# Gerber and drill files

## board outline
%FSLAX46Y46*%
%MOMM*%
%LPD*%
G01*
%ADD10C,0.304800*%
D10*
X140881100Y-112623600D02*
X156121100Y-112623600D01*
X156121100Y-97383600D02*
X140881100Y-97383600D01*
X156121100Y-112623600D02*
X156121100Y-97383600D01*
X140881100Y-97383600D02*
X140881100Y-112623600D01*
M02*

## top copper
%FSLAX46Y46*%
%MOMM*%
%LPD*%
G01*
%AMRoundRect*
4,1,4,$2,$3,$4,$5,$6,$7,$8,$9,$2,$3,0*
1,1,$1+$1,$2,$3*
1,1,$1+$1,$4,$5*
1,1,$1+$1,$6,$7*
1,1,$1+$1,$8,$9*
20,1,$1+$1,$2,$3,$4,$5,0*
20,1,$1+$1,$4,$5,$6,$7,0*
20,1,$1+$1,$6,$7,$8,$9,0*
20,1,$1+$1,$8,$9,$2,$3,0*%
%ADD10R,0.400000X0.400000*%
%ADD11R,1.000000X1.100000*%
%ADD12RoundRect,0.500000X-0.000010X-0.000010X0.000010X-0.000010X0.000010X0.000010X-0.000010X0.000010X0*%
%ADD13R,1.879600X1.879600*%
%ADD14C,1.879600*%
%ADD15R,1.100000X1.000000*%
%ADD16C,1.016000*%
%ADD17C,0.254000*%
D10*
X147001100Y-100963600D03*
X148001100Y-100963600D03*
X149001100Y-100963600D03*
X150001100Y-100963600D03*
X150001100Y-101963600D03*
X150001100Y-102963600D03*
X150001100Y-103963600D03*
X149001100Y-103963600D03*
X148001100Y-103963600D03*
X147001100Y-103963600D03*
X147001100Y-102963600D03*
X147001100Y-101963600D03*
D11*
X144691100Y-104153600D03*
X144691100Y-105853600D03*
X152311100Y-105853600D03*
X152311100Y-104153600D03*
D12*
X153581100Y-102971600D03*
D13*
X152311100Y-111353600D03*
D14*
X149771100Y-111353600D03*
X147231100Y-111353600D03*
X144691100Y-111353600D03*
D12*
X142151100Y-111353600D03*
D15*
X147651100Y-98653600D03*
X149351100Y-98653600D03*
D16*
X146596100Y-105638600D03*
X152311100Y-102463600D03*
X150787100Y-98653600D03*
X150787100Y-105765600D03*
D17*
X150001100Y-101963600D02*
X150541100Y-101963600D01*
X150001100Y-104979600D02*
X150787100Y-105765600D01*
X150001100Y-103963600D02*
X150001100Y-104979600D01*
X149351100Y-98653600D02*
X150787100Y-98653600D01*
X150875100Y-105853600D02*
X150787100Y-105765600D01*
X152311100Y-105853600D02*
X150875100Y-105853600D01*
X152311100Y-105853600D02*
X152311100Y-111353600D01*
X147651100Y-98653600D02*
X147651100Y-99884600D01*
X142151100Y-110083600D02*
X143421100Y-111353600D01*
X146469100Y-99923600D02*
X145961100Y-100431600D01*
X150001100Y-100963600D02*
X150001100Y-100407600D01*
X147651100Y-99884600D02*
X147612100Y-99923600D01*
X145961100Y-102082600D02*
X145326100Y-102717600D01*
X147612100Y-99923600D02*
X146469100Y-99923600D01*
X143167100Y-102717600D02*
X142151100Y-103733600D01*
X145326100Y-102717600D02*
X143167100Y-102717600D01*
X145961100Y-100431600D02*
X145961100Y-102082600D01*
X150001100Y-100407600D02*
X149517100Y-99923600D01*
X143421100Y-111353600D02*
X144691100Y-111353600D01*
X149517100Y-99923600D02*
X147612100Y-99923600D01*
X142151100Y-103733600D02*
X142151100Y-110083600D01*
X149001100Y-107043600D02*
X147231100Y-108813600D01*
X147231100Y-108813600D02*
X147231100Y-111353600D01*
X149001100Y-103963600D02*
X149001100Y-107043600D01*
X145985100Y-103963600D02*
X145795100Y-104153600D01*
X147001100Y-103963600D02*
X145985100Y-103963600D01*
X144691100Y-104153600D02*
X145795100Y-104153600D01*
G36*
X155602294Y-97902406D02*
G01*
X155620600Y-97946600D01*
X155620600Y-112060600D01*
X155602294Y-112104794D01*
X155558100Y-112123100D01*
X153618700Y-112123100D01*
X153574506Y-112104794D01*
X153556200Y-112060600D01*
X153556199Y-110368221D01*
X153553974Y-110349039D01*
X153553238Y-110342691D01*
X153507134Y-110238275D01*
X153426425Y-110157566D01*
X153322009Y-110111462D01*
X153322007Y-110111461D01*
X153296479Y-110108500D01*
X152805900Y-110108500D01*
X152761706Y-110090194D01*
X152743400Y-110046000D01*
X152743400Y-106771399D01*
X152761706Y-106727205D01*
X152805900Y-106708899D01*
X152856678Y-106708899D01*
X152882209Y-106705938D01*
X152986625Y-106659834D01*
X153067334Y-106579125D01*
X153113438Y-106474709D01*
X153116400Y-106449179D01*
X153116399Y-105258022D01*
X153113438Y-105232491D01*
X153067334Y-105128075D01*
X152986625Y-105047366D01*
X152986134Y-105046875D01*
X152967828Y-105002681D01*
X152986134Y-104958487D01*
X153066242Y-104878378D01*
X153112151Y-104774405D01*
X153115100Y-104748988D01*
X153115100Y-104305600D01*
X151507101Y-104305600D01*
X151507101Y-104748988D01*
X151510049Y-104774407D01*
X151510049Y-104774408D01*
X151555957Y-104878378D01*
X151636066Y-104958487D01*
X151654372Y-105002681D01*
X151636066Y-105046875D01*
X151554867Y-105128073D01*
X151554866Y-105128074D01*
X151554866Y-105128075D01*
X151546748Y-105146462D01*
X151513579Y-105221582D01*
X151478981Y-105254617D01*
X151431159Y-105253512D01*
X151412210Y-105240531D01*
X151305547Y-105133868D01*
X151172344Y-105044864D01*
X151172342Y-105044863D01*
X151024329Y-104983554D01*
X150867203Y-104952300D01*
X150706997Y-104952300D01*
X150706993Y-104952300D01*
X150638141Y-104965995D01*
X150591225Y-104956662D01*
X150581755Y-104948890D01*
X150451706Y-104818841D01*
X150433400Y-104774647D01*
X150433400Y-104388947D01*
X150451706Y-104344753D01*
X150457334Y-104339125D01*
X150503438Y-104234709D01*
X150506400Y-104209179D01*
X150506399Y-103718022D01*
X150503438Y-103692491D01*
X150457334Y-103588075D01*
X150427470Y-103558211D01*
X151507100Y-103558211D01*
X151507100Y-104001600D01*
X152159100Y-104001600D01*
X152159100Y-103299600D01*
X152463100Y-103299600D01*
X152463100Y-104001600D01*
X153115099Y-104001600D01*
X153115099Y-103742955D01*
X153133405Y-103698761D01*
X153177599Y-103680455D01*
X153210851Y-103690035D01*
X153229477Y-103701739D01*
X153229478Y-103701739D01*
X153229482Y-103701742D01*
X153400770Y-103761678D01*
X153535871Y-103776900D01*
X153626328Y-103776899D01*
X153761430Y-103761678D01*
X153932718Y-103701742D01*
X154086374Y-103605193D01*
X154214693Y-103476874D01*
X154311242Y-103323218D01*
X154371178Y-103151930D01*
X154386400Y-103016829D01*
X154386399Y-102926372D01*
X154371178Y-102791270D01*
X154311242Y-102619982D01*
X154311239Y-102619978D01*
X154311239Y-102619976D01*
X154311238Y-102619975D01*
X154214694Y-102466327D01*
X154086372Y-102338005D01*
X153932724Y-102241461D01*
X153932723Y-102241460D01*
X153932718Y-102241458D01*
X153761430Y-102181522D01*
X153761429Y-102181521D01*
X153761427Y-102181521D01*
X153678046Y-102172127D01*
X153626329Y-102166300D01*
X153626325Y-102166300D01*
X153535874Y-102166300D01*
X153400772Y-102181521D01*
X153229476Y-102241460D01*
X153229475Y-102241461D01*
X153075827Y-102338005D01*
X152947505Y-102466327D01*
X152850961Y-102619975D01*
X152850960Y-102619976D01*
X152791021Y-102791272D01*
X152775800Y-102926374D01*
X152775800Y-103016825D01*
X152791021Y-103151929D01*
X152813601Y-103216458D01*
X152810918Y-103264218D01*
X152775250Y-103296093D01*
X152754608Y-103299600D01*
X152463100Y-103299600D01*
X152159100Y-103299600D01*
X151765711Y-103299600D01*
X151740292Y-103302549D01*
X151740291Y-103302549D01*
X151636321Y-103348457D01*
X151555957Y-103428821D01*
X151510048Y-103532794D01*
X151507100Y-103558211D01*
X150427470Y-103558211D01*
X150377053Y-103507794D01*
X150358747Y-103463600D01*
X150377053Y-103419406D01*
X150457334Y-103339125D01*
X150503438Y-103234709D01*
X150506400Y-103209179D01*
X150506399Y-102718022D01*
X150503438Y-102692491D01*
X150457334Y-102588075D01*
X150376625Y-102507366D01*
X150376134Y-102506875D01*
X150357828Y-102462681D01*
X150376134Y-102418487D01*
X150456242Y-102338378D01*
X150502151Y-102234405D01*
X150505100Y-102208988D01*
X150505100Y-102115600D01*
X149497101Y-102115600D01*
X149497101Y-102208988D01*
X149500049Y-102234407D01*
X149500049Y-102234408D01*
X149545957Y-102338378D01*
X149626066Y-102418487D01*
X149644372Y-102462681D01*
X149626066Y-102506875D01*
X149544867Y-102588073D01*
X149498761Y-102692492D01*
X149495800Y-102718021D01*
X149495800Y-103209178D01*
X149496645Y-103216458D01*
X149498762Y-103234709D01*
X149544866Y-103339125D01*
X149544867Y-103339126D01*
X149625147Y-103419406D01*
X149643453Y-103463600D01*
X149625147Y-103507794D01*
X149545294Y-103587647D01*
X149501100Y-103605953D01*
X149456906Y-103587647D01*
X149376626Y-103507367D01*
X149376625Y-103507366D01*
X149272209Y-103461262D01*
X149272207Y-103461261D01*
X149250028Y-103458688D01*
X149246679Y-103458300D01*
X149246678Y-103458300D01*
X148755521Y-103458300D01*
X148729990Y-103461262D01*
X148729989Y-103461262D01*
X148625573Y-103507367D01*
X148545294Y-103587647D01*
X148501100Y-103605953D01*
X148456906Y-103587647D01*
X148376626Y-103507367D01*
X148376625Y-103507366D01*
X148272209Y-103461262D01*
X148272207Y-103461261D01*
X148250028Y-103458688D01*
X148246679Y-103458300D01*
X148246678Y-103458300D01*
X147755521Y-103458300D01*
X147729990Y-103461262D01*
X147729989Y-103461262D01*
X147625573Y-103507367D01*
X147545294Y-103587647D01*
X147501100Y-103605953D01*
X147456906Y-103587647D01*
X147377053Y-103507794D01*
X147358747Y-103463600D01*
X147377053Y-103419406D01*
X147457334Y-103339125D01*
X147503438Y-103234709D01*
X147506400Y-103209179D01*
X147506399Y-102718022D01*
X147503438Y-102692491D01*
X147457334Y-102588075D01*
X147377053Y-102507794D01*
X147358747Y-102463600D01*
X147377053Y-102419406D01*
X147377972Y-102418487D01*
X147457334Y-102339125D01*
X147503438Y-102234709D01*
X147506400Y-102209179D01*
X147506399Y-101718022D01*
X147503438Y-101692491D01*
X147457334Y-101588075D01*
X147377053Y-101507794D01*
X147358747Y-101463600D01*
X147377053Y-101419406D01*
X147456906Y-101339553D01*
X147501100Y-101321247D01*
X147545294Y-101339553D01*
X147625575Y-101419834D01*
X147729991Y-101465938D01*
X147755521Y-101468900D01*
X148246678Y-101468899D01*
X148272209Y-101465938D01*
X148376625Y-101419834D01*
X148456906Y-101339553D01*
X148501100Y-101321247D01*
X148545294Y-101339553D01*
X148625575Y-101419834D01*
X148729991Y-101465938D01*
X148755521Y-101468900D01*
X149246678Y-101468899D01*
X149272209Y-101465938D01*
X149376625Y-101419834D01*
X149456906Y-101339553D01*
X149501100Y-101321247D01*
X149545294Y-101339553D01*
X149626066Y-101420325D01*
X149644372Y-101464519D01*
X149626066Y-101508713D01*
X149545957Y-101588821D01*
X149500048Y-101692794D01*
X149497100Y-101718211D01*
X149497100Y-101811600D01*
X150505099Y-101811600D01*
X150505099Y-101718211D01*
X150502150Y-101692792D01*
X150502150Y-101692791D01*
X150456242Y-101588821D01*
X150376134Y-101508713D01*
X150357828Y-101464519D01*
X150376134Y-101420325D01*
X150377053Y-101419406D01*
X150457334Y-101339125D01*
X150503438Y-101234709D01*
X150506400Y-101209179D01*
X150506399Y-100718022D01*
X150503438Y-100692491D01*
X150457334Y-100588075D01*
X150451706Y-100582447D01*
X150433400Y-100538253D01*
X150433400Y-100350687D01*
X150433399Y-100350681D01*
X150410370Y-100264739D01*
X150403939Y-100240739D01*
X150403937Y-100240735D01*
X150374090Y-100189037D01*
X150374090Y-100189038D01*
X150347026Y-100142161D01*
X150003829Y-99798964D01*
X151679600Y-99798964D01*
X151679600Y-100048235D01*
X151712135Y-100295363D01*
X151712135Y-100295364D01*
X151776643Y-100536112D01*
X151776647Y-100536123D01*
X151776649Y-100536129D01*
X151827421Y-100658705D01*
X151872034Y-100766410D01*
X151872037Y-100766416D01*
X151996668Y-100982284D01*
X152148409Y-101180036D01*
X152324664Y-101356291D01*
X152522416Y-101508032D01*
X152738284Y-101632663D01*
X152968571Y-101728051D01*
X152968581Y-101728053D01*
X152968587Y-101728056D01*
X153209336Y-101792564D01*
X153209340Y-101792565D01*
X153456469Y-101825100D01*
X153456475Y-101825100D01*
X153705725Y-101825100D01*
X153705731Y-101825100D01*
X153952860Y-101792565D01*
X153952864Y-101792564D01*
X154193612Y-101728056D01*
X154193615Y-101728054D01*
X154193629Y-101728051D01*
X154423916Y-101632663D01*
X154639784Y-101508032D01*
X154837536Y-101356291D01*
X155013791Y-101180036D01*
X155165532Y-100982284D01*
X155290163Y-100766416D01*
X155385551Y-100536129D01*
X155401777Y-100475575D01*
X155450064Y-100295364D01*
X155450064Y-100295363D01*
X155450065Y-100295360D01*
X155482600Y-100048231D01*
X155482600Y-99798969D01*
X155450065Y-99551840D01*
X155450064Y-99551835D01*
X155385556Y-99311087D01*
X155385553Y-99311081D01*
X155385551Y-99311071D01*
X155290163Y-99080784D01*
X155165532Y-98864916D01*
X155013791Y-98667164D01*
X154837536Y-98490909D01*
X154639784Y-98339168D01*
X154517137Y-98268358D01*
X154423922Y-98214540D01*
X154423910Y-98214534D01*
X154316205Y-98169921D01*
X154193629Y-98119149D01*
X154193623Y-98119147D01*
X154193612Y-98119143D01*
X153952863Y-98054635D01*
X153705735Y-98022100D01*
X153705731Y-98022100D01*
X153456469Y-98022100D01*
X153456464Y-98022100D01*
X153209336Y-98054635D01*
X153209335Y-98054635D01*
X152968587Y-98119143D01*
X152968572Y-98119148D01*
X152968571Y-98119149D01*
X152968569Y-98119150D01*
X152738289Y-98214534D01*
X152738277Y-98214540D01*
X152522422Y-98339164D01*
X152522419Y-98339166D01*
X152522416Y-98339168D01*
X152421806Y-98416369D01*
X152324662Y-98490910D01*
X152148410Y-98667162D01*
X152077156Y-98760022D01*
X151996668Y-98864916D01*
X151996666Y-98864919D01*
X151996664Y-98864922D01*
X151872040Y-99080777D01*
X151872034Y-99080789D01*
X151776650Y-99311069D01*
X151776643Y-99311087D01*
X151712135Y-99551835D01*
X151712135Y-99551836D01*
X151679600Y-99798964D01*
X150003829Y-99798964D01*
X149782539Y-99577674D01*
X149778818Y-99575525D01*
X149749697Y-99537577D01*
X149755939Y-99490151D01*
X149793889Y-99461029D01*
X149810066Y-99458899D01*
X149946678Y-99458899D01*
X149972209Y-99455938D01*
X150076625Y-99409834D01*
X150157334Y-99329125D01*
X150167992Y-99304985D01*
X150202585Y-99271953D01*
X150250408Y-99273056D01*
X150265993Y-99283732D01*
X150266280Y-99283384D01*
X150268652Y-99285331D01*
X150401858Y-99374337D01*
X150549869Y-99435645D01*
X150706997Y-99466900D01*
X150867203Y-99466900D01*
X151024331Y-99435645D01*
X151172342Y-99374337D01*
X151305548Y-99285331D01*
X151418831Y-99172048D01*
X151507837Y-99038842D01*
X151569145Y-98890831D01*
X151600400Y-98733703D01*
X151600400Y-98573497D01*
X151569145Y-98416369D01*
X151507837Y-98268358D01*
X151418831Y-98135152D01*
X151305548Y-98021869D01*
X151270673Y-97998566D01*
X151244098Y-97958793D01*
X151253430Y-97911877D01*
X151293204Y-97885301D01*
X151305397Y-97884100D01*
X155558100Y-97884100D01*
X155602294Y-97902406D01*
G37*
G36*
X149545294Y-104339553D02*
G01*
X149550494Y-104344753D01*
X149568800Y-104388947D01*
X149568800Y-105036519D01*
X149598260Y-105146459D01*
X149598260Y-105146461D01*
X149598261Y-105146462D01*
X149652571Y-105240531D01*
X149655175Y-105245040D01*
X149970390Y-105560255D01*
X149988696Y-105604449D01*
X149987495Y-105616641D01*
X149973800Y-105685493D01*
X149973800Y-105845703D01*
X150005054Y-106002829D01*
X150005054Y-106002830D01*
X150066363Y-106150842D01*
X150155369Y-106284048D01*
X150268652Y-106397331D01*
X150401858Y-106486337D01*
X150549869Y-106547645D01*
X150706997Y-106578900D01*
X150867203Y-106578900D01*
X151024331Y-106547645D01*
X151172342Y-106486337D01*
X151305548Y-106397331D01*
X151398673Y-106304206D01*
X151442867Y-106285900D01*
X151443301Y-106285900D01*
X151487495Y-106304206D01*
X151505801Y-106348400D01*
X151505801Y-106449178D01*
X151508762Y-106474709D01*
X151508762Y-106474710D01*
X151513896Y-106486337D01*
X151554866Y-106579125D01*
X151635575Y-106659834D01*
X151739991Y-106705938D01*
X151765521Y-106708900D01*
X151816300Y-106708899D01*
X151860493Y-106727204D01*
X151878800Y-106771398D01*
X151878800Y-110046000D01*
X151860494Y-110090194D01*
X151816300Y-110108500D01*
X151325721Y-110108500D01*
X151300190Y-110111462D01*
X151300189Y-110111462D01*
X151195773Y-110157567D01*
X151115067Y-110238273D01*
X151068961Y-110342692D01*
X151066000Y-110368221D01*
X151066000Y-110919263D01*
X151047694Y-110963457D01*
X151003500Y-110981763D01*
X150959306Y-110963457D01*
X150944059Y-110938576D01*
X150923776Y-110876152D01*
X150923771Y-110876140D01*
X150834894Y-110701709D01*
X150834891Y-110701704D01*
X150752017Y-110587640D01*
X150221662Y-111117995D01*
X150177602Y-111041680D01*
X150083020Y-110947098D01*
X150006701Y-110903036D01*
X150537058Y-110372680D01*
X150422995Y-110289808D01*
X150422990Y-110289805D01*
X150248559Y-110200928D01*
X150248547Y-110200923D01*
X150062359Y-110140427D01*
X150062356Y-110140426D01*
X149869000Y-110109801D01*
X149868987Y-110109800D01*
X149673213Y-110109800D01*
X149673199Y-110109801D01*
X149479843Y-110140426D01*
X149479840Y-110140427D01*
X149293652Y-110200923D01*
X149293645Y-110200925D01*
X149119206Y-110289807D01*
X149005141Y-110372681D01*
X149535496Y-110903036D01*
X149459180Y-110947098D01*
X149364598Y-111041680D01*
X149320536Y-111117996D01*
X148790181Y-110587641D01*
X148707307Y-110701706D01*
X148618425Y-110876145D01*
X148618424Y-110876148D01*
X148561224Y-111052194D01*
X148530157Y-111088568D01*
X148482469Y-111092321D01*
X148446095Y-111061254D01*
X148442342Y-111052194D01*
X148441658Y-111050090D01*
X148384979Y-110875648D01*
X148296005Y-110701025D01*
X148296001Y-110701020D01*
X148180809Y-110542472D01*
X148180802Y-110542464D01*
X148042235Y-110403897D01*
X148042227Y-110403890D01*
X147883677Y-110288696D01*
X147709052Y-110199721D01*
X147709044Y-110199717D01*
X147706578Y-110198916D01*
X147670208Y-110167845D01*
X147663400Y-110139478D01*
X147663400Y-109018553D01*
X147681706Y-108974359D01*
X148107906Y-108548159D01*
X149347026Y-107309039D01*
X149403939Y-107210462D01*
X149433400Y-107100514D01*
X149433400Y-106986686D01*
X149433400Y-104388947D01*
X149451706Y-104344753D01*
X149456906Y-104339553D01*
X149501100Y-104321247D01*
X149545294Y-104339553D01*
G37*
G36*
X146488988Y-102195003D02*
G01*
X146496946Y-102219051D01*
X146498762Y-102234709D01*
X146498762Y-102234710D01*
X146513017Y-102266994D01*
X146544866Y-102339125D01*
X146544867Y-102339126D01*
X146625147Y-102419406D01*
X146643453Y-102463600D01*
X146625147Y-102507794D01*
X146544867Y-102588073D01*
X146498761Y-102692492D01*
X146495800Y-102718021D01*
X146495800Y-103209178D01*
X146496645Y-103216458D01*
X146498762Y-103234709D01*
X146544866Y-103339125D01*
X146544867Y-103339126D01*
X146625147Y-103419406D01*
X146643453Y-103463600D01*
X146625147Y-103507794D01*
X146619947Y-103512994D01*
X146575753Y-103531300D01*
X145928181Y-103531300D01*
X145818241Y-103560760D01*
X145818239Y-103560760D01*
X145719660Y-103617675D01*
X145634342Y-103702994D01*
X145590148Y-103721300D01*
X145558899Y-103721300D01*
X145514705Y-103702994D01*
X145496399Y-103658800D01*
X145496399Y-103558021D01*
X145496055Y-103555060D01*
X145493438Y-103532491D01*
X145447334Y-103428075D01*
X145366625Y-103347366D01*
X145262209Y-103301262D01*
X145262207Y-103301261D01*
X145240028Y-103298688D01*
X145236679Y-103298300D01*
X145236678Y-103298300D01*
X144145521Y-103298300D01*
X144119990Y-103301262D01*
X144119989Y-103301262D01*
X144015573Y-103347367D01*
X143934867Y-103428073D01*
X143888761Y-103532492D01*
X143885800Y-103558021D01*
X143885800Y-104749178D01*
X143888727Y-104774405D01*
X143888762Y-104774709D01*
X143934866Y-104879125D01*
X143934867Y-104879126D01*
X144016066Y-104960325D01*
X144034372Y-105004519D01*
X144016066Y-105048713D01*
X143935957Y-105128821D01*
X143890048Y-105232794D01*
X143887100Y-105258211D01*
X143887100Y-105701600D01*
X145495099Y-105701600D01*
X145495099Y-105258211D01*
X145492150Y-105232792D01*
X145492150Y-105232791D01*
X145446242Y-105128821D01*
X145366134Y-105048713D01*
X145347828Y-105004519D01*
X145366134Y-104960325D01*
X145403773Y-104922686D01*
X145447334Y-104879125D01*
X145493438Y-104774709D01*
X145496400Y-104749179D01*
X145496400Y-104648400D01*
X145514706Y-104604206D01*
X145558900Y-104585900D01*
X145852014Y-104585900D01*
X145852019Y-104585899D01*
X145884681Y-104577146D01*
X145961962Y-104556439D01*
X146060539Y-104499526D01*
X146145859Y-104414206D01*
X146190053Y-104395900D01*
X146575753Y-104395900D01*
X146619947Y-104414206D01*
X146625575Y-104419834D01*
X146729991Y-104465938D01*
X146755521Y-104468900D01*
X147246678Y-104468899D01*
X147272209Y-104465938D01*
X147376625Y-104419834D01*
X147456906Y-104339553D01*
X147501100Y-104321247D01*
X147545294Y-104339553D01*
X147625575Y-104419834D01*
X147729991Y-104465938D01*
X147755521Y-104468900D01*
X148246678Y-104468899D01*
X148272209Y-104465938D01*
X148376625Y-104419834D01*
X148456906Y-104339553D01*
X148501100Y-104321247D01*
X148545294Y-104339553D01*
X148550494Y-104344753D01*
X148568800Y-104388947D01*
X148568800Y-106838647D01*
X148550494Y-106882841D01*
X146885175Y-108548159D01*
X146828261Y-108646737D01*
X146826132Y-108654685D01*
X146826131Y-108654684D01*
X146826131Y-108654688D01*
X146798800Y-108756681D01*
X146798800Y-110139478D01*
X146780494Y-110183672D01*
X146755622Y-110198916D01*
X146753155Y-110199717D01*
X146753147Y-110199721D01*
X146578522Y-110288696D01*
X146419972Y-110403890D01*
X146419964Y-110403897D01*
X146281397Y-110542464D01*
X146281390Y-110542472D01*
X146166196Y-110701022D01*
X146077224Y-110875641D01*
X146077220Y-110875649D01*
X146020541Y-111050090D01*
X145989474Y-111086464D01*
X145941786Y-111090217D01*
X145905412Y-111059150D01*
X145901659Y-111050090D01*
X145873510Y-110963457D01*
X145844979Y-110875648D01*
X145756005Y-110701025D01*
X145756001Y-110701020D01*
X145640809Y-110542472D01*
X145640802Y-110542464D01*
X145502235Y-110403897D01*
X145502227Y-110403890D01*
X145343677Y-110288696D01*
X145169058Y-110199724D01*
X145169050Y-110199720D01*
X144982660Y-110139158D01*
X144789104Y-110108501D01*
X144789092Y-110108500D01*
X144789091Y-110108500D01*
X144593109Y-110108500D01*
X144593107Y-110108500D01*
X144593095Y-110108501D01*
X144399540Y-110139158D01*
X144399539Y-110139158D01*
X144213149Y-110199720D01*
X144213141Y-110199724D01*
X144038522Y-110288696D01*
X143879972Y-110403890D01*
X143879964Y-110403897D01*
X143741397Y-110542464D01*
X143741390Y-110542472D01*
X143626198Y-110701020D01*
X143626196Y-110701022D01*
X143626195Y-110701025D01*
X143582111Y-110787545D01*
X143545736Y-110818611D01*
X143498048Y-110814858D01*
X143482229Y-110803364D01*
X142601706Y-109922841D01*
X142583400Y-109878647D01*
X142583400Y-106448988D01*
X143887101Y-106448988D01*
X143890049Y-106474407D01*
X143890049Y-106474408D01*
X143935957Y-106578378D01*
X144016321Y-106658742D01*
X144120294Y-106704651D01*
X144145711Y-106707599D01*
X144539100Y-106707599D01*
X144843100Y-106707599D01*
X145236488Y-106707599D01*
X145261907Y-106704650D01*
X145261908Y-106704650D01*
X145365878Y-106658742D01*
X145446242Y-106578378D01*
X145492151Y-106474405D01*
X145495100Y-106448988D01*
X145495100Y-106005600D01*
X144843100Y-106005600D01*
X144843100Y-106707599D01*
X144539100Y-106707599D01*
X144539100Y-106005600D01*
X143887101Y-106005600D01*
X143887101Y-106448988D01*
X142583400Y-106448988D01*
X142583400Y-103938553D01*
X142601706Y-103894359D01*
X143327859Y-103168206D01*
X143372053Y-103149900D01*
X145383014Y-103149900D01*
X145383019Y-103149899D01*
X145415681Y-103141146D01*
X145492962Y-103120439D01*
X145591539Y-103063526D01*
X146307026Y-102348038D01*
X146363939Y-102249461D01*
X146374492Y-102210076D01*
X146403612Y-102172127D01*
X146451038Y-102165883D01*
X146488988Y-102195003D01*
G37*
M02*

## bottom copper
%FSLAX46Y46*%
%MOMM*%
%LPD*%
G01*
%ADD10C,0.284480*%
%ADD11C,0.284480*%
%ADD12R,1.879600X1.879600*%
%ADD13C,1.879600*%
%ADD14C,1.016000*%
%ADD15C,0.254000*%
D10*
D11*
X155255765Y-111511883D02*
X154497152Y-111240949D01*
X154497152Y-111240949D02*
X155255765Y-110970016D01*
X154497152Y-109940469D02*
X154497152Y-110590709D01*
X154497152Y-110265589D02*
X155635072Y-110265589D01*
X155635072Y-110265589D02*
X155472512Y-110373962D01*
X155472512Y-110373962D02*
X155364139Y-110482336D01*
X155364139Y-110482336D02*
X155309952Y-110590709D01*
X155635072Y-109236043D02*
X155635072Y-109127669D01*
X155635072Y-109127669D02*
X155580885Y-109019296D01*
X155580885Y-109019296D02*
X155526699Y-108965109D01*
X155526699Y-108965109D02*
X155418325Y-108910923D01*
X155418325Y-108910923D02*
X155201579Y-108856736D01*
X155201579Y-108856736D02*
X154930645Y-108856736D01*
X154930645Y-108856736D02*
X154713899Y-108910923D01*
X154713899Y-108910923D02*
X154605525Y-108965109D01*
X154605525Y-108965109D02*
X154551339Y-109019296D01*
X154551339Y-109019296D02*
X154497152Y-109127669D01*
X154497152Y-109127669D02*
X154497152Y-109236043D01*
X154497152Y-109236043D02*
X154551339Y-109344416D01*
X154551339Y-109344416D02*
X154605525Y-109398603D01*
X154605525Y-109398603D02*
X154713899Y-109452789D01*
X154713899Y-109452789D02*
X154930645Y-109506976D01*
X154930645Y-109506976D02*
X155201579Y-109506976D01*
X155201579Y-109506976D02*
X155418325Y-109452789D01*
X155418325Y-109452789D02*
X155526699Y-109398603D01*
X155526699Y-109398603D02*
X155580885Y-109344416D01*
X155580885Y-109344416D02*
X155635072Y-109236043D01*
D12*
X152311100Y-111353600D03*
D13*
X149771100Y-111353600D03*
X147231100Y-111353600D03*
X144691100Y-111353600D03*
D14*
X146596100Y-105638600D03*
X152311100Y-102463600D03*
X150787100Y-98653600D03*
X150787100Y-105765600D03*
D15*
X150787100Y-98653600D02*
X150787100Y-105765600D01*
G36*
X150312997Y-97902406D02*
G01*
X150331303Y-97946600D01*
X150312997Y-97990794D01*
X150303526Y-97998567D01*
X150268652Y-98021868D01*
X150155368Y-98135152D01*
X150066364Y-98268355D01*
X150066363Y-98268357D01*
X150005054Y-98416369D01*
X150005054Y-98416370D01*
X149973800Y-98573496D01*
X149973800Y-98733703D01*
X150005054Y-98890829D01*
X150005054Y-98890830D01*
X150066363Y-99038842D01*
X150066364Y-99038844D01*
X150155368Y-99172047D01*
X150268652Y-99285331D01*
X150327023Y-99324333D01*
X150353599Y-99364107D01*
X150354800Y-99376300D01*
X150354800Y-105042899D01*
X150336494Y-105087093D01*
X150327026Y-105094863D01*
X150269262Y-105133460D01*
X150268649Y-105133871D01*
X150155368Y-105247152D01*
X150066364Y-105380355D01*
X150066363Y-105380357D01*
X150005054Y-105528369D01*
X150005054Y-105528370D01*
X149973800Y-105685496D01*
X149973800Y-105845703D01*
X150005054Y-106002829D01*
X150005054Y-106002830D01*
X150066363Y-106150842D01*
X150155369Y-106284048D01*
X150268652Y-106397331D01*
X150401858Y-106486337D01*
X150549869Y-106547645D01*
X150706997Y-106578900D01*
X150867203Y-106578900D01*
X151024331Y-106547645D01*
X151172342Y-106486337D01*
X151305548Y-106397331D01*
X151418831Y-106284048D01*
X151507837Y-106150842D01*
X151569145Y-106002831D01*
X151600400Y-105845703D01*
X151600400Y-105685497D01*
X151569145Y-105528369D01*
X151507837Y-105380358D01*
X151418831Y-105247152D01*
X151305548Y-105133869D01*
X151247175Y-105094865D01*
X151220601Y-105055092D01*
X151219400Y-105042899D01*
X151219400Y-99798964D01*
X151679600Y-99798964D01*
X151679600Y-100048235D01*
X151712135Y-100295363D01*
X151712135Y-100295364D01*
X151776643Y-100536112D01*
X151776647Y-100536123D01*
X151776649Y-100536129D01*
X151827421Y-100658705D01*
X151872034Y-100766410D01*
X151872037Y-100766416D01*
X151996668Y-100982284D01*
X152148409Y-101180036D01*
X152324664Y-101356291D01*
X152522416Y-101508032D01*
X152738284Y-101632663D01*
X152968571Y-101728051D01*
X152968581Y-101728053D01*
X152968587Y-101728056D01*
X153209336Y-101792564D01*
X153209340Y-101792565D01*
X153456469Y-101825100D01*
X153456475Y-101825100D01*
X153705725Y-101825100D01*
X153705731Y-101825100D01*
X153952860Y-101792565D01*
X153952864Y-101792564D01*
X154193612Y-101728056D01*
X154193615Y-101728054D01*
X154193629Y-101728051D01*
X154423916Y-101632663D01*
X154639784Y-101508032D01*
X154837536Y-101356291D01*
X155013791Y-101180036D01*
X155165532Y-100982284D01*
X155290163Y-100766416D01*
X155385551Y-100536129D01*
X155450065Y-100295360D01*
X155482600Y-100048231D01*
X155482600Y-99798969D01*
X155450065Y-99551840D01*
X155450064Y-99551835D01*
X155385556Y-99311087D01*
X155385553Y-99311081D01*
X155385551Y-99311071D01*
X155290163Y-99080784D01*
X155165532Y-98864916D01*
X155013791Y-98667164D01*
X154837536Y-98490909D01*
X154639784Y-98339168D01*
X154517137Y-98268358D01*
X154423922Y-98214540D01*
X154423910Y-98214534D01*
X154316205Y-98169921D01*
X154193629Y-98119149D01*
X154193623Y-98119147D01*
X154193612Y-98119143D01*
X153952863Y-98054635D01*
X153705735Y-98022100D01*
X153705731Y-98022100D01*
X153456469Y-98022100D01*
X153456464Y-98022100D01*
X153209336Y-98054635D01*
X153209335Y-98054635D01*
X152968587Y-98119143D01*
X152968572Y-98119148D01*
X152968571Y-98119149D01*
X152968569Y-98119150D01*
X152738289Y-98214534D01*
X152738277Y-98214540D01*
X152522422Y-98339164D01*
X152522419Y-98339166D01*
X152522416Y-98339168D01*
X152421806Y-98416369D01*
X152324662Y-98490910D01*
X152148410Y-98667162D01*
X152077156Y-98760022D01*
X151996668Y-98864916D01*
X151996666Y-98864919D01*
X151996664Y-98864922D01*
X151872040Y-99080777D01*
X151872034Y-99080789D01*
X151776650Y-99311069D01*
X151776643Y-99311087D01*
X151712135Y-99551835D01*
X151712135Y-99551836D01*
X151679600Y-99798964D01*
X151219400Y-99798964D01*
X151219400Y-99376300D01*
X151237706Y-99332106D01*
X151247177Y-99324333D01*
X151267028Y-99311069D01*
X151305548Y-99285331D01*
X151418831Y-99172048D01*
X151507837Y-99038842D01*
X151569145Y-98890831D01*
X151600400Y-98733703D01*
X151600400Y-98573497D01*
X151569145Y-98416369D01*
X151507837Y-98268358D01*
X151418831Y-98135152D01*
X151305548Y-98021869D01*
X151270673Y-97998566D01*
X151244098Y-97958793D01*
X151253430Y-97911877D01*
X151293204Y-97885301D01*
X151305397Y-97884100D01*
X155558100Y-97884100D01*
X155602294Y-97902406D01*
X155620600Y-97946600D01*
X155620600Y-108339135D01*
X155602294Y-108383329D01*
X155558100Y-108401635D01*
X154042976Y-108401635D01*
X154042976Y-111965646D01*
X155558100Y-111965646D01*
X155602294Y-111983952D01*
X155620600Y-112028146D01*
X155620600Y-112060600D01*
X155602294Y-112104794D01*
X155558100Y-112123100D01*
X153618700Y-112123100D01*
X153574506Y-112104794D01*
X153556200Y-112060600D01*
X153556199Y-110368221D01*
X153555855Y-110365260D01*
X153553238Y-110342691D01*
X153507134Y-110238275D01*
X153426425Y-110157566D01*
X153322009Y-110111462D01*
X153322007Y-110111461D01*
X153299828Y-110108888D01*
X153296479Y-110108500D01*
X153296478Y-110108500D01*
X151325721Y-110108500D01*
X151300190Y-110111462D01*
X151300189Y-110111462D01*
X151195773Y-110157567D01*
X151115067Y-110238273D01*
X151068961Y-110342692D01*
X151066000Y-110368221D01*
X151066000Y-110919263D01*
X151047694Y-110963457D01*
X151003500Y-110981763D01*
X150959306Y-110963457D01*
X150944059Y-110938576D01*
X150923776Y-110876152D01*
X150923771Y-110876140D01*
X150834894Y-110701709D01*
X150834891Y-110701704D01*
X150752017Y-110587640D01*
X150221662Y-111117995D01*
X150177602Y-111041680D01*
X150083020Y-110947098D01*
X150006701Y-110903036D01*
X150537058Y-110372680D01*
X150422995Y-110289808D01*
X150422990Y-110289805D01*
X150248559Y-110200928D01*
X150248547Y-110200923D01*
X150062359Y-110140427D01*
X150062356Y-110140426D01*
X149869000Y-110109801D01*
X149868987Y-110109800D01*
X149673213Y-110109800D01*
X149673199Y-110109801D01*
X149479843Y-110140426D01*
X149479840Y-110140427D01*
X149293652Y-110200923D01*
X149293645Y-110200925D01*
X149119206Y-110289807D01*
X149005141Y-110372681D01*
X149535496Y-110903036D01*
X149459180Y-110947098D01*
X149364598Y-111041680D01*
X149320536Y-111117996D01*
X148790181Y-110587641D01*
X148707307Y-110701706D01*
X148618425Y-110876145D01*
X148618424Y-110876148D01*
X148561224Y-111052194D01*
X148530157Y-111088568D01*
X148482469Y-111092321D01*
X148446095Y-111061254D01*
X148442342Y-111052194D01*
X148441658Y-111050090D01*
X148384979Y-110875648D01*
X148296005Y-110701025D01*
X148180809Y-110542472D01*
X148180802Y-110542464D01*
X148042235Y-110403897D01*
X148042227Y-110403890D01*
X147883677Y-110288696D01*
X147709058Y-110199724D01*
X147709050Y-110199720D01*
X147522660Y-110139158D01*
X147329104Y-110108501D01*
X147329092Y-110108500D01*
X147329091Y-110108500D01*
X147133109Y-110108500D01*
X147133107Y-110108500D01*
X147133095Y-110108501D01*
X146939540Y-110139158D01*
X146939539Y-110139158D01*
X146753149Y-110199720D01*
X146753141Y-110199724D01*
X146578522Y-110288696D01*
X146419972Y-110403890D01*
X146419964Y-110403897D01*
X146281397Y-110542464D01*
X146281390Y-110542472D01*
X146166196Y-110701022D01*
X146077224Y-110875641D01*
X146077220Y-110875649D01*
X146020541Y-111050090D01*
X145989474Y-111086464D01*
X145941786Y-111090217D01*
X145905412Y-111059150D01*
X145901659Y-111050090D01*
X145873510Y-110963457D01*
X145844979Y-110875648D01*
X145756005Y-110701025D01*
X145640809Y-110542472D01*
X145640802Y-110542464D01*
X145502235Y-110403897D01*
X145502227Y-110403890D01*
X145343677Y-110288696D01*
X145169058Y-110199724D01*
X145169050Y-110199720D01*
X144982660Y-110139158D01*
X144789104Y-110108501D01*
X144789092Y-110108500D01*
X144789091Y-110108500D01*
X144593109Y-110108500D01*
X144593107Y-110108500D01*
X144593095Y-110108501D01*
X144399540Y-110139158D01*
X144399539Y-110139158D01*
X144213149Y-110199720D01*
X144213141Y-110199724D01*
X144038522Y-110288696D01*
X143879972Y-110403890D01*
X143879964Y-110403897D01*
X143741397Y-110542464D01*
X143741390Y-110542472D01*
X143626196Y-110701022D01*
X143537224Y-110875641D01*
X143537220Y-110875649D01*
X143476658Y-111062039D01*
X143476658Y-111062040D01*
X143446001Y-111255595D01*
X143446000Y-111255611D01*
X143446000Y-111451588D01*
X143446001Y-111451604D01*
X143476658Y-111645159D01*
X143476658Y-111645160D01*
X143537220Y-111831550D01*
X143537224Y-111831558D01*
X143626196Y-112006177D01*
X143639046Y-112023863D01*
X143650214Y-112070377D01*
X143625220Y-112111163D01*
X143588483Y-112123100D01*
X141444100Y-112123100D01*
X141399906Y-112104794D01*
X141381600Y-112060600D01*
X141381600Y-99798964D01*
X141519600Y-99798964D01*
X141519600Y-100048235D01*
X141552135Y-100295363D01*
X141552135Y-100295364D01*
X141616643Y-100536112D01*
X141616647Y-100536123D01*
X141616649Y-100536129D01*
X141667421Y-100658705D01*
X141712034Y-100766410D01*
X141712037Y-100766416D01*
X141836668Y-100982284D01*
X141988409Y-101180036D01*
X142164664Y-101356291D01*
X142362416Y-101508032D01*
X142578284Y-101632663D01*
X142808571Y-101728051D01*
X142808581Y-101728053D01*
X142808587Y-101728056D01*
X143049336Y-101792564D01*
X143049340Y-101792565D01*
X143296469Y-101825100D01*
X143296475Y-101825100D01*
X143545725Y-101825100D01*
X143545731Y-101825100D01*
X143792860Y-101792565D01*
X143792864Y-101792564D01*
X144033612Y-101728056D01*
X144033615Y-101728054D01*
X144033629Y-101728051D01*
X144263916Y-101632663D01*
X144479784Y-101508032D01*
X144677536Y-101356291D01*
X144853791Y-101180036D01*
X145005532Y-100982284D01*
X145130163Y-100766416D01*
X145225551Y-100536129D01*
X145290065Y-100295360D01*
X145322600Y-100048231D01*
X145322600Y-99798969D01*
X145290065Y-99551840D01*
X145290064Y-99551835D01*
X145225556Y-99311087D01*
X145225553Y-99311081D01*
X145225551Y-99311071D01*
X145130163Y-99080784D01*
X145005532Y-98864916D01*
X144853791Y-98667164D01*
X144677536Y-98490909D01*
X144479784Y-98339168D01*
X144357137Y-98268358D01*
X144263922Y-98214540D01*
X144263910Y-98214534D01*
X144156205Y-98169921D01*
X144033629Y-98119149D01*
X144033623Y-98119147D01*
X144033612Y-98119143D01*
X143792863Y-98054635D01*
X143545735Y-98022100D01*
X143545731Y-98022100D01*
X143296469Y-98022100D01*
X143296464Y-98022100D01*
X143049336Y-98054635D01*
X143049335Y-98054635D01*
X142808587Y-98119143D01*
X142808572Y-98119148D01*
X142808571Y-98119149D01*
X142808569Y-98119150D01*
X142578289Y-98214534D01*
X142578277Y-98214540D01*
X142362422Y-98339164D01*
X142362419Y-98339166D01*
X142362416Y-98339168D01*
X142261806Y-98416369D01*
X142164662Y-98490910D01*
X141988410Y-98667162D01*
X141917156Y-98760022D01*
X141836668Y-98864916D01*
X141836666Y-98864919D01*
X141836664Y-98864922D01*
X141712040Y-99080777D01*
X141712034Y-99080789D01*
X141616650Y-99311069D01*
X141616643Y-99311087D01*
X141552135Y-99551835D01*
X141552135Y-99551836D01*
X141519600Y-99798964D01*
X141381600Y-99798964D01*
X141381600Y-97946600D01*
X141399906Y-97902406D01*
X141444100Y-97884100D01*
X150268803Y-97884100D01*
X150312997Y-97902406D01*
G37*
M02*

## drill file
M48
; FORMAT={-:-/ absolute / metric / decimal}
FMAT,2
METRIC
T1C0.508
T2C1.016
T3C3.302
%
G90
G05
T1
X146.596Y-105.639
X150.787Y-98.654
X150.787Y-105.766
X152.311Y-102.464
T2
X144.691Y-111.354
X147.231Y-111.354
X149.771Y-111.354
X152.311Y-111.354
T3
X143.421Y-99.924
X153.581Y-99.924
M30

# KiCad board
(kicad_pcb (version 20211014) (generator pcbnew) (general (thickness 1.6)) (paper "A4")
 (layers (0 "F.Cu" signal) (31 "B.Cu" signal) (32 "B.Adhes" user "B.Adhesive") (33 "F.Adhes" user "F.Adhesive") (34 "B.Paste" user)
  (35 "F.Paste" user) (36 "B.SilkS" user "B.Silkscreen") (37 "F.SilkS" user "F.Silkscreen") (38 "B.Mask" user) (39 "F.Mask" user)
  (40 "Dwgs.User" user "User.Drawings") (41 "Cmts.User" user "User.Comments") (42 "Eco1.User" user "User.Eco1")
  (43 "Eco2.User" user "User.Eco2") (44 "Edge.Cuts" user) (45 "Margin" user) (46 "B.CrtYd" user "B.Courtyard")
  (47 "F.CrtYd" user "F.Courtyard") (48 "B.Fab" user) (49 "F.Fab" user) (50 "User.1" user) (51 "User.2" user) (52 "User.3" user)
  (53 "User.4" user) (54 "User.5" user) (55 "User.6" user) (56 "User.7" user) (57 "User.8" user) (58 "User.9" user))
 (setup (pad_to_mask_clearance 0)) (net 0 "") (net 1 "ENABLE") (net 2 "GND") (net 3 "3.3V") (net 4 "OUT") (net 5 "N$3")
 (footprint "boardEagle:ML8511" (layer "F.Cu") (at 148.5011 102.4636 -90)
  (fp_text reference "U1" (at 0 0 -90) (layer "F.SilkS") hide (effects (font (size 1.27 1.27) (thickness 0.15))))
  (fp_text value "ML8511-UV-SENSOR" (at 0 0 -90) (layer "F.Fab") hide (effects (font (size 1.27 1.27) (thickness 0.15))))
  (pad "1" smd rect (at -1.5 1.5 270) (size 0.4 0.4) (layers "F.Cu" "F.Paste" "F.Mask") (solder_mask_margin 0.1016))
  (pad "2" smd rect (at -1.5 0.5 270) (size 0.4 0.4) (layers "F.Cu" "F.Paste" "F.Mask") (solder_mask_margin 0.1016))
  (pad "3" smd rect (at -1.5 -0.5 270) (size 0.4 0.4) (layers "F.Cu" "F.Paste" "F.Mask") (solder_mask_margin 0.1016))
  (pad "4" smd rect (at -1.5 -1.5 270) (size 0.4 0.4) (layers "F.Cu" "F.Paste" "F.Mask") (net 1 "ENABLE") (solder_mask_margin 0.1016))
  (pad "5" smd rect (at -0.5 -1.5 270) (size 0.4 0.4) (layers "F.Cu" "F.Paste" "F.Mask") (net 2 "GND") (solder_mask_margin 0.1016))
  (pad "6" smd rect (at 0.5 -1.5 270) (size 0.4 0.4) (layers "F.Cu" "F.Paste" "F.Mask") (solder_mask_margin 0.1016))
  (pad "7" smd rect (at 1.5 -1.5 270) (size 0.4 0.4) (layers "F.Cu" "F.Paste" "F.Mask") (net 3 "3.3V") (solder_mask_margin 0.1016))
  (pad "8" smd rect (at 1.5 -0.5 270) (size 0.4 0.4) (layers "F.Cu" "F.Paste" "F.Mask") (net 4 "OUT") (solder_mask_margin 0.1016))
  (pad "9" smd rect (at 1.5 0.5 270) (size 0.4 0.4) (layers "F.Cu" "F.Paste" "F.Mask") (solder_mask_margin 0.1016))
  (pad "10" smd rect (at 1.5 1.5 270) (size 0.4 0.4) (layers "F.Cu" "F.Paste" "F.Mask") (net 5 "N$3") (solder_mask_margin 0.1016))
  (pad "11" smd rect (at 0.5 1.5 270) (size 0.4 0.4) (layers "F.Cu" "F.Paste" "F.Mask") (solder_mask_margin 0.1016))
  (pad "12" smd rect (at -0.5 1.5 270) (size 0.4 0.4) (layers "F.Cu" "F.Paste" "F.Mask") (solder_mask_margin 0.1016)))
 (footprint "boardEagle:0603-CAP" (layer "F.Cu") (at 144.6911 105.0036 -90)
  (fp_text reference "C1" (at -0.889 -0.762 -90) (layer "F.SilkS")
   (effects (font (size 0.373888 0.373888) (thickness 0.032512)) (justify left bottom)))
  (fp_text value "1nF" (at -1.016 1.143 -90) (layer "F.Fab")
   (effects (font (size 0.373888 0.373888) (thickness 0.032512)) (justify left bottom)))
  (pad "1" smd rect (at -0.85 0 270) (size 1.1 1) (layers "F.Cu" "F.Paste" "F.Mask") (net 5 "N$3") (solder_mask_margin 0.1016))
  (pad "2" smd rect (at 0.85 0 270) (size 1.1 1) (layers "F.Cu" "F.Paste" "F.Mask") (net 2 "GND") (solder_mask_margin 0.1016)))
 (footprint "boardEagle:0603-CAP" (layer "F.Cu") (at 152.3111 105.0036 90)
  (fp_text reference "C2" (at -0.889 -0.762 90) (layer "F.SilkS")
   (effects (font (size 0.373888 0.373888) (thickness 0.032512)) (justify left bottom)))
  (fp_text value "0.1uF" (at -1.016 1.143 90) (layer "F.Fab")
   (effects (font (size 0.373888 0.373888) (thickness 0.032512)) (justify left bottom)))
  (pad "1" smd rect (at -0.85 0 90) (size 1.1 1) (layers "F.Cu" "F.Paste" "F.Mask") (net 3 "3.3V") (solder_mask_margin 0.1016))
  (pad "2" smd rect (at 0.85 0 90) (size 1.1 1) (layers "F.Cu" "F.Paste" "F.Mask") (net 2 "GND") (solder_mask_margin 0.1016)))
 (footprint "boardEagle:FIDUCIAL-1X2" (layer "F.Cu") (at 153.5811 102.9716)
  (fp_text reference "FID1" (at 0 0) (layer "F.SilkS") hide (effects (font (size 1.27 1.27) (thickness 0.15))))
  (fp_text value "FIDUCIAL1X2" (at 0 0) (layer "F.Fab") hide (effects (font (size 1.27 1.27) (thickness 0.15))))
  (pad "1" smd roundrect (at 0 0) (size 1 1) (layers "F.Cu" "F.Mask") (roundrect_rratio 0.5) (solder_mask_margin 0.1016)))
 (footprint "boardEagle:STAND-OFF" (layer "F.Cu") (at 153.5811 99.9236)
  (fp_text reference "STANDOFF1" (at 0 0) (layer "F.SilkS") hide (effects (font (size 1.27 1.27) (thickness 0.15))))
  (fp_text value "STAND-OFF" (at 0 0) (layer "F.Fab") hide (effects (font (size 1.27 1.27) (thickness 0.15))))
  (pad "" np_thru_hole circle (at 0 0) (size 3.302 3.302) (drill 3.302) (layers *.Cu *.Mask)))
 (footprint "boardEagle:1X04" (layer "F.Cu") (at 152.3111 111.3536 180)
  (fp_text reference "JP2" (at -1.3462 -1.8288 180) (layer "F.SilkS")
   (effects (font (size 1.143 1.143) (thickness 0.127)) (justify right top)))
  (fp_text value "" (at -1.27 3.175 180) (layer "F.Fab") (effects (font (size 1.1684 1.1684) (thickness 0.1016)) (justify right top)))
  (pad "1" thru_hole rect (at 0 0 270) (size 1.8796 1.8796) (drill 1.016) (layers *.Cu *.Mask) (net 3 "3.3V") (solder_mask_margin 0.1016))
  (pad "2" thru_hole circle (at 2.54 0 270) (size 1.8796 1.8796) (drill 1.016) (layers *.Cu *.Mask) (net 2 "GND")
   (solder_mask_margin 0.1016))
  (pad "3" thru_hole circle (at 5.08 0 270) (size 1.8796 1.8796) (drill 1.016) (layers *.Cu *.Mask) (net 4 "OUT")
   (solder_mask_margin 0.1016))
  (pad "4" thru_hole circle (at 7.62 0 270) (size 1.8796 1.8796) (drill 1.016) (layers *.Cu *.Mask) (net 1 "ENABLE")
   (solder_mask_margin 0.1016)))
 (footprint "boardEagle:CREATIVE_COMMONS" (layer "F.Cu") (at 125.6411 122.7836)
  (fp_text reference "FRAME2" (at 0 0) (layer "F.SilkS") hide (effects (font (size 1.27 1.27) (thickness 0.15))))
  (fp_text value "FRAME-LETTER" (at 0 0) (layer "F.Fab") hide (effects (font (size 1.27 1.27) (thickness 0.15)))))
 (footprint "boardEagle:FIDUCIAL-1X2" (layer "F.Cu") (at 142.1511 111.3536)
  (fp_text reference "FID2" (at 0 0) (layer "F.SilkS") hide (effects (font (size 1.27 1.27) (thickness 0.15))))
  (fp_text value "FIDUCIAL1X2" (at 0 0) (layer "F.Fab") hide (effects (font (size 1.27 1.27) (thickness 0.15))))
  (pad "1" smd roundrect (at 0 0) (size 1 1) (layers "F.Cu" "F.Mask") (roundrect_rratio 0.5) (solder_mask_margin 0.1016)))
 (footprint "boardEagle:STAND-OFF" (layer "F.Cu") (at 143.4211 99.9236)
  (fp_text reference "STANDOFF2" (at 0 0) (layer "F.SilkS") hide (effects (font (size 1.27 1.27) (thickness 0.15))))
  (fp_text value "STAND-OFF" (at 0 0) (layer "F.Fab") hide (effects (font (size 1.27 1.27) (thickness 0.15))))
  (pad "" np_thru_hole circle (at 0 0) (size 3.302 3.302) (drill 3.302) (layers *.Cu *.Mask)))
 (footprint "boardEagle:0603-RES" (layer "F.Cu") (at 148.5011 98.6536)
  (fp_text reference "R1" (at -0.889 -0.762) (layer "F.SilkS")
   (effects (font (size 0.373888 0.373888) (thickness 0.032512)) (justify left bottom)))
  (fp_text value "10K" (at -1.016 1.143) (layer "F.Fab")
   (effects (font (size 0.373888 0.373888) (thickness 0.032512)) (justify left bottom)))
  (pad "1" smd rect (at -0.85 0) (size 1.1 1) (layers "F.Cu" "F.Paste" "F.Mask") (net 1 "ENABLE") (solder_mask_margin 0.1016))
  (pad "2" smd rect (at 0.85 0) (size 1.1 1) (layers "F.Cu" "F.Paste" "F.Mask") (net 3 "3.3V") (solder_mask_margin 0.1016)))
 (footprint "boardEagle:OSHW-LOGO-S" (layer "B.Cu") (at 149.5171 100.3046 180)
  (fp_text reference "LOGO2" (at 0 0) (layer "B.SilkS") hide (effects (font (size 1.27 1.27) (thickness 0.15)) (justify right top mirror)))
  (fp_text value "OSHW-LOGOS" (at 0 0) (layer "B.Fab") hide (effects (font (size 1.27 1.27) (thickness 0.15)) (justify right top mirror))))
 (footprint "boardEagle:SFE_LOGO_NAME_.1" (layer "B.Cu") (at 154.4701 106.2736 180)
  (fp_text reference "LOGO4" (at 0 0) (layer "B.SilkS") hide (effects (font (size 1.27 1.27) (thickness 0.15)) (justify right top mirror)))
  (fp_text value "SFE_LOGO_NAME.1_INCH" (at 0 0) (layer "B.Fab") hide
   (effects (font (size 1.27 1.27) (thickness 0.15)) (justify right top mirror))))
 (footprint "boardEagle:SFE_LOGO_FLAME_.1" (layer "B.Cu") (at 147.7391 101.8286 180)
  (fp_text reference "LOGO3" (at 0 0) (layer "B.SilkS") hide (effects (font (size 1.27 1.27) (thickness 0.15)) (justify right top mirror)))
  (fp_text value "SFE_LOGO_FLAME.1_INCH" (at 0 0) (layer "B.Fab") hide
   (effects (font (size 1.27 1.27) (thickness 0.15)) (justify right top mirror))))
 (gr_line (start 140.8811 112.6236) (end 156.1211 112.6236) (layer "Edge.Cuts") (width 0.3048))
 (gr_line (start 156.1211 97.3836) (end 140.8811 97.3836) (layer "Edge.Cuts") (width 0.3048))
 (gr_line (start 156.1211 112.6236) (end 156.1211 97.3836) (layer "Edge.Cuts") (width 0.3048))
 (gr_line (start 140.8811 97.3836) (end 140.8811 112.6236) (layer "Edge.Cuts") (width 0.3048))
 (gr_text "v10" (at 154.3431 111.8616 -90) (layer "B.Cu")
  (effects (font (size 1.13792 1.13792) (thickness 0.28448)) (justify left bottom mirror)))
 (segment (start 150.0011 101.9636) (end 150.5411 101.9636) (width 0.254) (layer "F.Cu") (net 2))
 (via (at 146.5961 105.6386) (size 1.016) (drill 0.508) (layers "F.Cu" "B.Cu") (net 2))
 (via (at 152.3111 102.4636) (size 1.016) (drill 0.508) (layers "F.Cu" "B.Cu") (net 2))
 (segment (start 150.0011 104.9796) (end 150.7871 105.7656) (width 0.254) (layer "F.Cu") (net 3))
 (segment (start 150.0011 103.9636) (end 150.0011 104.9796) (width 0.254) (layer "F.Cu") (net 3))
 (segment (start 149.3511 98.6536) (end 150.7871 98.6536) (width 0.254) (layer "F.Cu") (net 3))
 (segment (start 150.8751 105.8536) (end 150.7871 105.7656) (width 0.254) (layer "F.Cu") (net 3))
 (segment (start 152.3111 105.8536) (end 150.8751 105.8536) (width 0.254) (layer "F.Cu") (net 3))
 (segment (start 152.3111 105.8536) (end 152.3111 111.3536) (width 0.254) (layer "F.Cu") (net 3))
 (via (at 150.7871 98.6536) (size 1.016) (drill 0.508) (layers "F.Cu" "B.Cu") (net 3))
 (via (at 150.7871 105.7656) (size 1.016) (drill 0.508) (layers "F.Cu" "B.Cu") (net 3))
 (segment (start 150.7871 98.6536) (end 150.7871 105.7656) (width 0.254) (layer "B.Cu") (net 3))
 (segment (start 147.6511 98.6536) (end 147.6511 99.8846) (width 0.254) (layer "F.Cu") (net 1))
 (segment (start 142.1511 110.0836) (end 143.4211 111.3536) (width 0.254) (layer "F.Cu") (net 1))
 (segment (start 146.4691 99.9236) (end 145.9611 100.4316) (width 0.254) (layer "F.Cu") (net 1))
 (segment (start 150.0011 100.9636) (end 150.0011 100.4076) (width 0.254) (layer "F.Cu") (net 1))
 (segment (start 147.6511 99.8846) (end 147.6121 99.9236) (width 0.254) (layer "F.Cu") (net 1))
 (segment (start 145.9611 102.0826) (end 145.3261 102.7176) (width 0.254) (layer "F.Cu") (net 1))
 (segment (start 147.6121 99.9236) (end 146.4691 99.9236) (width 0.254) (layer "F.Cu") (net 1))
 (segment (start 143.1671 102.7176) (end 142.1511 103.7336) (width 0.254) (layer "F.Cu") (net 1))
 (segment (start 145.3261 102.7176) (end 143.1671 102.7176) (width 0.254) (layer "F.Cu") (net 1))
 (segment (start 145.9611 100.4316) (end 145.9611 102.0826) (width 0.254) (layer "F.Cu") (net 1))
 (segment (start 150.0011 100.4076) (end 149.5171 99.9236) (width 0.254) (layer "F.Cu") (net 1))
 (segment (start 143.4211 111.3536) (end 144.6911 111.3536) (width 0.254) (layer "F.Cu") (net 1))
 (segment (start 149.5171 99.9236) (end 147.6121 99.9236) (width 0.254) (layer "F.Cu") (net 1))
 (segment (start 142.1511 103.7336) (end 142.1511 110.0836) (width 0.254) (layer "F.Cu") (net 1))
 (segment (start 149.0011 107.0436) (end 147.2311 108.8136) (width 0.254) (layer "F.Cu") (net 4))
 (segment (start 147.2311 108.8136) (end 147.2311 111.3536) (width 0.254) (layer "F.Cu") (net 4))
 (segment (start 149.0011 103.9636) (end 149.0011 107.0436) (width 0.254) (layer "F.Cu") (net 4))
 (segment (start 145.9851 103.9636) (end 145.7951 104.1536) (width 0.254) (layer "F.Cu") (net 5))
 (segment (start 147.0011 103.9636) (end 145.9851 103.9636) (width 0.254) (layer "F.Cu") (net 5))
 (segment (start 144.6911 104.1536) (end 145.7951 104.1536) (width 0.254) (layer "F.Cu") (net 5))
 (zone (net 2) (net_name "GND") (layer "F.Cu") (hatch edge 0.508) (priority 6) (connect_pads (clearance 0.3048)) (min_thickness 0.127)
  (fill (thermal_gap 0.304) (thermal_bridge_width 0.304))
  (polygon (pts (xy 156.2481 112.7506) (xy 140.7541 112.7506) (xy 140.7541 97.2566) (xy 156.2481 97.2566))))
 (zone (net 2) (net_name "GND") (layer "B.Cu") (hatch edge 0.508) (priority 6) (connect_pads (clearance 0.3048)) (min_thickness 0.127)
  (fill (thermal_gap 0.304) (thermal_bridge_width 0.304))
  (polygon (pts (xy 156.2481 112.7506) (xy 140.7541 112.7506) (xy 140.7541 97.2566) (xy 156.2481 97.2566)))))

